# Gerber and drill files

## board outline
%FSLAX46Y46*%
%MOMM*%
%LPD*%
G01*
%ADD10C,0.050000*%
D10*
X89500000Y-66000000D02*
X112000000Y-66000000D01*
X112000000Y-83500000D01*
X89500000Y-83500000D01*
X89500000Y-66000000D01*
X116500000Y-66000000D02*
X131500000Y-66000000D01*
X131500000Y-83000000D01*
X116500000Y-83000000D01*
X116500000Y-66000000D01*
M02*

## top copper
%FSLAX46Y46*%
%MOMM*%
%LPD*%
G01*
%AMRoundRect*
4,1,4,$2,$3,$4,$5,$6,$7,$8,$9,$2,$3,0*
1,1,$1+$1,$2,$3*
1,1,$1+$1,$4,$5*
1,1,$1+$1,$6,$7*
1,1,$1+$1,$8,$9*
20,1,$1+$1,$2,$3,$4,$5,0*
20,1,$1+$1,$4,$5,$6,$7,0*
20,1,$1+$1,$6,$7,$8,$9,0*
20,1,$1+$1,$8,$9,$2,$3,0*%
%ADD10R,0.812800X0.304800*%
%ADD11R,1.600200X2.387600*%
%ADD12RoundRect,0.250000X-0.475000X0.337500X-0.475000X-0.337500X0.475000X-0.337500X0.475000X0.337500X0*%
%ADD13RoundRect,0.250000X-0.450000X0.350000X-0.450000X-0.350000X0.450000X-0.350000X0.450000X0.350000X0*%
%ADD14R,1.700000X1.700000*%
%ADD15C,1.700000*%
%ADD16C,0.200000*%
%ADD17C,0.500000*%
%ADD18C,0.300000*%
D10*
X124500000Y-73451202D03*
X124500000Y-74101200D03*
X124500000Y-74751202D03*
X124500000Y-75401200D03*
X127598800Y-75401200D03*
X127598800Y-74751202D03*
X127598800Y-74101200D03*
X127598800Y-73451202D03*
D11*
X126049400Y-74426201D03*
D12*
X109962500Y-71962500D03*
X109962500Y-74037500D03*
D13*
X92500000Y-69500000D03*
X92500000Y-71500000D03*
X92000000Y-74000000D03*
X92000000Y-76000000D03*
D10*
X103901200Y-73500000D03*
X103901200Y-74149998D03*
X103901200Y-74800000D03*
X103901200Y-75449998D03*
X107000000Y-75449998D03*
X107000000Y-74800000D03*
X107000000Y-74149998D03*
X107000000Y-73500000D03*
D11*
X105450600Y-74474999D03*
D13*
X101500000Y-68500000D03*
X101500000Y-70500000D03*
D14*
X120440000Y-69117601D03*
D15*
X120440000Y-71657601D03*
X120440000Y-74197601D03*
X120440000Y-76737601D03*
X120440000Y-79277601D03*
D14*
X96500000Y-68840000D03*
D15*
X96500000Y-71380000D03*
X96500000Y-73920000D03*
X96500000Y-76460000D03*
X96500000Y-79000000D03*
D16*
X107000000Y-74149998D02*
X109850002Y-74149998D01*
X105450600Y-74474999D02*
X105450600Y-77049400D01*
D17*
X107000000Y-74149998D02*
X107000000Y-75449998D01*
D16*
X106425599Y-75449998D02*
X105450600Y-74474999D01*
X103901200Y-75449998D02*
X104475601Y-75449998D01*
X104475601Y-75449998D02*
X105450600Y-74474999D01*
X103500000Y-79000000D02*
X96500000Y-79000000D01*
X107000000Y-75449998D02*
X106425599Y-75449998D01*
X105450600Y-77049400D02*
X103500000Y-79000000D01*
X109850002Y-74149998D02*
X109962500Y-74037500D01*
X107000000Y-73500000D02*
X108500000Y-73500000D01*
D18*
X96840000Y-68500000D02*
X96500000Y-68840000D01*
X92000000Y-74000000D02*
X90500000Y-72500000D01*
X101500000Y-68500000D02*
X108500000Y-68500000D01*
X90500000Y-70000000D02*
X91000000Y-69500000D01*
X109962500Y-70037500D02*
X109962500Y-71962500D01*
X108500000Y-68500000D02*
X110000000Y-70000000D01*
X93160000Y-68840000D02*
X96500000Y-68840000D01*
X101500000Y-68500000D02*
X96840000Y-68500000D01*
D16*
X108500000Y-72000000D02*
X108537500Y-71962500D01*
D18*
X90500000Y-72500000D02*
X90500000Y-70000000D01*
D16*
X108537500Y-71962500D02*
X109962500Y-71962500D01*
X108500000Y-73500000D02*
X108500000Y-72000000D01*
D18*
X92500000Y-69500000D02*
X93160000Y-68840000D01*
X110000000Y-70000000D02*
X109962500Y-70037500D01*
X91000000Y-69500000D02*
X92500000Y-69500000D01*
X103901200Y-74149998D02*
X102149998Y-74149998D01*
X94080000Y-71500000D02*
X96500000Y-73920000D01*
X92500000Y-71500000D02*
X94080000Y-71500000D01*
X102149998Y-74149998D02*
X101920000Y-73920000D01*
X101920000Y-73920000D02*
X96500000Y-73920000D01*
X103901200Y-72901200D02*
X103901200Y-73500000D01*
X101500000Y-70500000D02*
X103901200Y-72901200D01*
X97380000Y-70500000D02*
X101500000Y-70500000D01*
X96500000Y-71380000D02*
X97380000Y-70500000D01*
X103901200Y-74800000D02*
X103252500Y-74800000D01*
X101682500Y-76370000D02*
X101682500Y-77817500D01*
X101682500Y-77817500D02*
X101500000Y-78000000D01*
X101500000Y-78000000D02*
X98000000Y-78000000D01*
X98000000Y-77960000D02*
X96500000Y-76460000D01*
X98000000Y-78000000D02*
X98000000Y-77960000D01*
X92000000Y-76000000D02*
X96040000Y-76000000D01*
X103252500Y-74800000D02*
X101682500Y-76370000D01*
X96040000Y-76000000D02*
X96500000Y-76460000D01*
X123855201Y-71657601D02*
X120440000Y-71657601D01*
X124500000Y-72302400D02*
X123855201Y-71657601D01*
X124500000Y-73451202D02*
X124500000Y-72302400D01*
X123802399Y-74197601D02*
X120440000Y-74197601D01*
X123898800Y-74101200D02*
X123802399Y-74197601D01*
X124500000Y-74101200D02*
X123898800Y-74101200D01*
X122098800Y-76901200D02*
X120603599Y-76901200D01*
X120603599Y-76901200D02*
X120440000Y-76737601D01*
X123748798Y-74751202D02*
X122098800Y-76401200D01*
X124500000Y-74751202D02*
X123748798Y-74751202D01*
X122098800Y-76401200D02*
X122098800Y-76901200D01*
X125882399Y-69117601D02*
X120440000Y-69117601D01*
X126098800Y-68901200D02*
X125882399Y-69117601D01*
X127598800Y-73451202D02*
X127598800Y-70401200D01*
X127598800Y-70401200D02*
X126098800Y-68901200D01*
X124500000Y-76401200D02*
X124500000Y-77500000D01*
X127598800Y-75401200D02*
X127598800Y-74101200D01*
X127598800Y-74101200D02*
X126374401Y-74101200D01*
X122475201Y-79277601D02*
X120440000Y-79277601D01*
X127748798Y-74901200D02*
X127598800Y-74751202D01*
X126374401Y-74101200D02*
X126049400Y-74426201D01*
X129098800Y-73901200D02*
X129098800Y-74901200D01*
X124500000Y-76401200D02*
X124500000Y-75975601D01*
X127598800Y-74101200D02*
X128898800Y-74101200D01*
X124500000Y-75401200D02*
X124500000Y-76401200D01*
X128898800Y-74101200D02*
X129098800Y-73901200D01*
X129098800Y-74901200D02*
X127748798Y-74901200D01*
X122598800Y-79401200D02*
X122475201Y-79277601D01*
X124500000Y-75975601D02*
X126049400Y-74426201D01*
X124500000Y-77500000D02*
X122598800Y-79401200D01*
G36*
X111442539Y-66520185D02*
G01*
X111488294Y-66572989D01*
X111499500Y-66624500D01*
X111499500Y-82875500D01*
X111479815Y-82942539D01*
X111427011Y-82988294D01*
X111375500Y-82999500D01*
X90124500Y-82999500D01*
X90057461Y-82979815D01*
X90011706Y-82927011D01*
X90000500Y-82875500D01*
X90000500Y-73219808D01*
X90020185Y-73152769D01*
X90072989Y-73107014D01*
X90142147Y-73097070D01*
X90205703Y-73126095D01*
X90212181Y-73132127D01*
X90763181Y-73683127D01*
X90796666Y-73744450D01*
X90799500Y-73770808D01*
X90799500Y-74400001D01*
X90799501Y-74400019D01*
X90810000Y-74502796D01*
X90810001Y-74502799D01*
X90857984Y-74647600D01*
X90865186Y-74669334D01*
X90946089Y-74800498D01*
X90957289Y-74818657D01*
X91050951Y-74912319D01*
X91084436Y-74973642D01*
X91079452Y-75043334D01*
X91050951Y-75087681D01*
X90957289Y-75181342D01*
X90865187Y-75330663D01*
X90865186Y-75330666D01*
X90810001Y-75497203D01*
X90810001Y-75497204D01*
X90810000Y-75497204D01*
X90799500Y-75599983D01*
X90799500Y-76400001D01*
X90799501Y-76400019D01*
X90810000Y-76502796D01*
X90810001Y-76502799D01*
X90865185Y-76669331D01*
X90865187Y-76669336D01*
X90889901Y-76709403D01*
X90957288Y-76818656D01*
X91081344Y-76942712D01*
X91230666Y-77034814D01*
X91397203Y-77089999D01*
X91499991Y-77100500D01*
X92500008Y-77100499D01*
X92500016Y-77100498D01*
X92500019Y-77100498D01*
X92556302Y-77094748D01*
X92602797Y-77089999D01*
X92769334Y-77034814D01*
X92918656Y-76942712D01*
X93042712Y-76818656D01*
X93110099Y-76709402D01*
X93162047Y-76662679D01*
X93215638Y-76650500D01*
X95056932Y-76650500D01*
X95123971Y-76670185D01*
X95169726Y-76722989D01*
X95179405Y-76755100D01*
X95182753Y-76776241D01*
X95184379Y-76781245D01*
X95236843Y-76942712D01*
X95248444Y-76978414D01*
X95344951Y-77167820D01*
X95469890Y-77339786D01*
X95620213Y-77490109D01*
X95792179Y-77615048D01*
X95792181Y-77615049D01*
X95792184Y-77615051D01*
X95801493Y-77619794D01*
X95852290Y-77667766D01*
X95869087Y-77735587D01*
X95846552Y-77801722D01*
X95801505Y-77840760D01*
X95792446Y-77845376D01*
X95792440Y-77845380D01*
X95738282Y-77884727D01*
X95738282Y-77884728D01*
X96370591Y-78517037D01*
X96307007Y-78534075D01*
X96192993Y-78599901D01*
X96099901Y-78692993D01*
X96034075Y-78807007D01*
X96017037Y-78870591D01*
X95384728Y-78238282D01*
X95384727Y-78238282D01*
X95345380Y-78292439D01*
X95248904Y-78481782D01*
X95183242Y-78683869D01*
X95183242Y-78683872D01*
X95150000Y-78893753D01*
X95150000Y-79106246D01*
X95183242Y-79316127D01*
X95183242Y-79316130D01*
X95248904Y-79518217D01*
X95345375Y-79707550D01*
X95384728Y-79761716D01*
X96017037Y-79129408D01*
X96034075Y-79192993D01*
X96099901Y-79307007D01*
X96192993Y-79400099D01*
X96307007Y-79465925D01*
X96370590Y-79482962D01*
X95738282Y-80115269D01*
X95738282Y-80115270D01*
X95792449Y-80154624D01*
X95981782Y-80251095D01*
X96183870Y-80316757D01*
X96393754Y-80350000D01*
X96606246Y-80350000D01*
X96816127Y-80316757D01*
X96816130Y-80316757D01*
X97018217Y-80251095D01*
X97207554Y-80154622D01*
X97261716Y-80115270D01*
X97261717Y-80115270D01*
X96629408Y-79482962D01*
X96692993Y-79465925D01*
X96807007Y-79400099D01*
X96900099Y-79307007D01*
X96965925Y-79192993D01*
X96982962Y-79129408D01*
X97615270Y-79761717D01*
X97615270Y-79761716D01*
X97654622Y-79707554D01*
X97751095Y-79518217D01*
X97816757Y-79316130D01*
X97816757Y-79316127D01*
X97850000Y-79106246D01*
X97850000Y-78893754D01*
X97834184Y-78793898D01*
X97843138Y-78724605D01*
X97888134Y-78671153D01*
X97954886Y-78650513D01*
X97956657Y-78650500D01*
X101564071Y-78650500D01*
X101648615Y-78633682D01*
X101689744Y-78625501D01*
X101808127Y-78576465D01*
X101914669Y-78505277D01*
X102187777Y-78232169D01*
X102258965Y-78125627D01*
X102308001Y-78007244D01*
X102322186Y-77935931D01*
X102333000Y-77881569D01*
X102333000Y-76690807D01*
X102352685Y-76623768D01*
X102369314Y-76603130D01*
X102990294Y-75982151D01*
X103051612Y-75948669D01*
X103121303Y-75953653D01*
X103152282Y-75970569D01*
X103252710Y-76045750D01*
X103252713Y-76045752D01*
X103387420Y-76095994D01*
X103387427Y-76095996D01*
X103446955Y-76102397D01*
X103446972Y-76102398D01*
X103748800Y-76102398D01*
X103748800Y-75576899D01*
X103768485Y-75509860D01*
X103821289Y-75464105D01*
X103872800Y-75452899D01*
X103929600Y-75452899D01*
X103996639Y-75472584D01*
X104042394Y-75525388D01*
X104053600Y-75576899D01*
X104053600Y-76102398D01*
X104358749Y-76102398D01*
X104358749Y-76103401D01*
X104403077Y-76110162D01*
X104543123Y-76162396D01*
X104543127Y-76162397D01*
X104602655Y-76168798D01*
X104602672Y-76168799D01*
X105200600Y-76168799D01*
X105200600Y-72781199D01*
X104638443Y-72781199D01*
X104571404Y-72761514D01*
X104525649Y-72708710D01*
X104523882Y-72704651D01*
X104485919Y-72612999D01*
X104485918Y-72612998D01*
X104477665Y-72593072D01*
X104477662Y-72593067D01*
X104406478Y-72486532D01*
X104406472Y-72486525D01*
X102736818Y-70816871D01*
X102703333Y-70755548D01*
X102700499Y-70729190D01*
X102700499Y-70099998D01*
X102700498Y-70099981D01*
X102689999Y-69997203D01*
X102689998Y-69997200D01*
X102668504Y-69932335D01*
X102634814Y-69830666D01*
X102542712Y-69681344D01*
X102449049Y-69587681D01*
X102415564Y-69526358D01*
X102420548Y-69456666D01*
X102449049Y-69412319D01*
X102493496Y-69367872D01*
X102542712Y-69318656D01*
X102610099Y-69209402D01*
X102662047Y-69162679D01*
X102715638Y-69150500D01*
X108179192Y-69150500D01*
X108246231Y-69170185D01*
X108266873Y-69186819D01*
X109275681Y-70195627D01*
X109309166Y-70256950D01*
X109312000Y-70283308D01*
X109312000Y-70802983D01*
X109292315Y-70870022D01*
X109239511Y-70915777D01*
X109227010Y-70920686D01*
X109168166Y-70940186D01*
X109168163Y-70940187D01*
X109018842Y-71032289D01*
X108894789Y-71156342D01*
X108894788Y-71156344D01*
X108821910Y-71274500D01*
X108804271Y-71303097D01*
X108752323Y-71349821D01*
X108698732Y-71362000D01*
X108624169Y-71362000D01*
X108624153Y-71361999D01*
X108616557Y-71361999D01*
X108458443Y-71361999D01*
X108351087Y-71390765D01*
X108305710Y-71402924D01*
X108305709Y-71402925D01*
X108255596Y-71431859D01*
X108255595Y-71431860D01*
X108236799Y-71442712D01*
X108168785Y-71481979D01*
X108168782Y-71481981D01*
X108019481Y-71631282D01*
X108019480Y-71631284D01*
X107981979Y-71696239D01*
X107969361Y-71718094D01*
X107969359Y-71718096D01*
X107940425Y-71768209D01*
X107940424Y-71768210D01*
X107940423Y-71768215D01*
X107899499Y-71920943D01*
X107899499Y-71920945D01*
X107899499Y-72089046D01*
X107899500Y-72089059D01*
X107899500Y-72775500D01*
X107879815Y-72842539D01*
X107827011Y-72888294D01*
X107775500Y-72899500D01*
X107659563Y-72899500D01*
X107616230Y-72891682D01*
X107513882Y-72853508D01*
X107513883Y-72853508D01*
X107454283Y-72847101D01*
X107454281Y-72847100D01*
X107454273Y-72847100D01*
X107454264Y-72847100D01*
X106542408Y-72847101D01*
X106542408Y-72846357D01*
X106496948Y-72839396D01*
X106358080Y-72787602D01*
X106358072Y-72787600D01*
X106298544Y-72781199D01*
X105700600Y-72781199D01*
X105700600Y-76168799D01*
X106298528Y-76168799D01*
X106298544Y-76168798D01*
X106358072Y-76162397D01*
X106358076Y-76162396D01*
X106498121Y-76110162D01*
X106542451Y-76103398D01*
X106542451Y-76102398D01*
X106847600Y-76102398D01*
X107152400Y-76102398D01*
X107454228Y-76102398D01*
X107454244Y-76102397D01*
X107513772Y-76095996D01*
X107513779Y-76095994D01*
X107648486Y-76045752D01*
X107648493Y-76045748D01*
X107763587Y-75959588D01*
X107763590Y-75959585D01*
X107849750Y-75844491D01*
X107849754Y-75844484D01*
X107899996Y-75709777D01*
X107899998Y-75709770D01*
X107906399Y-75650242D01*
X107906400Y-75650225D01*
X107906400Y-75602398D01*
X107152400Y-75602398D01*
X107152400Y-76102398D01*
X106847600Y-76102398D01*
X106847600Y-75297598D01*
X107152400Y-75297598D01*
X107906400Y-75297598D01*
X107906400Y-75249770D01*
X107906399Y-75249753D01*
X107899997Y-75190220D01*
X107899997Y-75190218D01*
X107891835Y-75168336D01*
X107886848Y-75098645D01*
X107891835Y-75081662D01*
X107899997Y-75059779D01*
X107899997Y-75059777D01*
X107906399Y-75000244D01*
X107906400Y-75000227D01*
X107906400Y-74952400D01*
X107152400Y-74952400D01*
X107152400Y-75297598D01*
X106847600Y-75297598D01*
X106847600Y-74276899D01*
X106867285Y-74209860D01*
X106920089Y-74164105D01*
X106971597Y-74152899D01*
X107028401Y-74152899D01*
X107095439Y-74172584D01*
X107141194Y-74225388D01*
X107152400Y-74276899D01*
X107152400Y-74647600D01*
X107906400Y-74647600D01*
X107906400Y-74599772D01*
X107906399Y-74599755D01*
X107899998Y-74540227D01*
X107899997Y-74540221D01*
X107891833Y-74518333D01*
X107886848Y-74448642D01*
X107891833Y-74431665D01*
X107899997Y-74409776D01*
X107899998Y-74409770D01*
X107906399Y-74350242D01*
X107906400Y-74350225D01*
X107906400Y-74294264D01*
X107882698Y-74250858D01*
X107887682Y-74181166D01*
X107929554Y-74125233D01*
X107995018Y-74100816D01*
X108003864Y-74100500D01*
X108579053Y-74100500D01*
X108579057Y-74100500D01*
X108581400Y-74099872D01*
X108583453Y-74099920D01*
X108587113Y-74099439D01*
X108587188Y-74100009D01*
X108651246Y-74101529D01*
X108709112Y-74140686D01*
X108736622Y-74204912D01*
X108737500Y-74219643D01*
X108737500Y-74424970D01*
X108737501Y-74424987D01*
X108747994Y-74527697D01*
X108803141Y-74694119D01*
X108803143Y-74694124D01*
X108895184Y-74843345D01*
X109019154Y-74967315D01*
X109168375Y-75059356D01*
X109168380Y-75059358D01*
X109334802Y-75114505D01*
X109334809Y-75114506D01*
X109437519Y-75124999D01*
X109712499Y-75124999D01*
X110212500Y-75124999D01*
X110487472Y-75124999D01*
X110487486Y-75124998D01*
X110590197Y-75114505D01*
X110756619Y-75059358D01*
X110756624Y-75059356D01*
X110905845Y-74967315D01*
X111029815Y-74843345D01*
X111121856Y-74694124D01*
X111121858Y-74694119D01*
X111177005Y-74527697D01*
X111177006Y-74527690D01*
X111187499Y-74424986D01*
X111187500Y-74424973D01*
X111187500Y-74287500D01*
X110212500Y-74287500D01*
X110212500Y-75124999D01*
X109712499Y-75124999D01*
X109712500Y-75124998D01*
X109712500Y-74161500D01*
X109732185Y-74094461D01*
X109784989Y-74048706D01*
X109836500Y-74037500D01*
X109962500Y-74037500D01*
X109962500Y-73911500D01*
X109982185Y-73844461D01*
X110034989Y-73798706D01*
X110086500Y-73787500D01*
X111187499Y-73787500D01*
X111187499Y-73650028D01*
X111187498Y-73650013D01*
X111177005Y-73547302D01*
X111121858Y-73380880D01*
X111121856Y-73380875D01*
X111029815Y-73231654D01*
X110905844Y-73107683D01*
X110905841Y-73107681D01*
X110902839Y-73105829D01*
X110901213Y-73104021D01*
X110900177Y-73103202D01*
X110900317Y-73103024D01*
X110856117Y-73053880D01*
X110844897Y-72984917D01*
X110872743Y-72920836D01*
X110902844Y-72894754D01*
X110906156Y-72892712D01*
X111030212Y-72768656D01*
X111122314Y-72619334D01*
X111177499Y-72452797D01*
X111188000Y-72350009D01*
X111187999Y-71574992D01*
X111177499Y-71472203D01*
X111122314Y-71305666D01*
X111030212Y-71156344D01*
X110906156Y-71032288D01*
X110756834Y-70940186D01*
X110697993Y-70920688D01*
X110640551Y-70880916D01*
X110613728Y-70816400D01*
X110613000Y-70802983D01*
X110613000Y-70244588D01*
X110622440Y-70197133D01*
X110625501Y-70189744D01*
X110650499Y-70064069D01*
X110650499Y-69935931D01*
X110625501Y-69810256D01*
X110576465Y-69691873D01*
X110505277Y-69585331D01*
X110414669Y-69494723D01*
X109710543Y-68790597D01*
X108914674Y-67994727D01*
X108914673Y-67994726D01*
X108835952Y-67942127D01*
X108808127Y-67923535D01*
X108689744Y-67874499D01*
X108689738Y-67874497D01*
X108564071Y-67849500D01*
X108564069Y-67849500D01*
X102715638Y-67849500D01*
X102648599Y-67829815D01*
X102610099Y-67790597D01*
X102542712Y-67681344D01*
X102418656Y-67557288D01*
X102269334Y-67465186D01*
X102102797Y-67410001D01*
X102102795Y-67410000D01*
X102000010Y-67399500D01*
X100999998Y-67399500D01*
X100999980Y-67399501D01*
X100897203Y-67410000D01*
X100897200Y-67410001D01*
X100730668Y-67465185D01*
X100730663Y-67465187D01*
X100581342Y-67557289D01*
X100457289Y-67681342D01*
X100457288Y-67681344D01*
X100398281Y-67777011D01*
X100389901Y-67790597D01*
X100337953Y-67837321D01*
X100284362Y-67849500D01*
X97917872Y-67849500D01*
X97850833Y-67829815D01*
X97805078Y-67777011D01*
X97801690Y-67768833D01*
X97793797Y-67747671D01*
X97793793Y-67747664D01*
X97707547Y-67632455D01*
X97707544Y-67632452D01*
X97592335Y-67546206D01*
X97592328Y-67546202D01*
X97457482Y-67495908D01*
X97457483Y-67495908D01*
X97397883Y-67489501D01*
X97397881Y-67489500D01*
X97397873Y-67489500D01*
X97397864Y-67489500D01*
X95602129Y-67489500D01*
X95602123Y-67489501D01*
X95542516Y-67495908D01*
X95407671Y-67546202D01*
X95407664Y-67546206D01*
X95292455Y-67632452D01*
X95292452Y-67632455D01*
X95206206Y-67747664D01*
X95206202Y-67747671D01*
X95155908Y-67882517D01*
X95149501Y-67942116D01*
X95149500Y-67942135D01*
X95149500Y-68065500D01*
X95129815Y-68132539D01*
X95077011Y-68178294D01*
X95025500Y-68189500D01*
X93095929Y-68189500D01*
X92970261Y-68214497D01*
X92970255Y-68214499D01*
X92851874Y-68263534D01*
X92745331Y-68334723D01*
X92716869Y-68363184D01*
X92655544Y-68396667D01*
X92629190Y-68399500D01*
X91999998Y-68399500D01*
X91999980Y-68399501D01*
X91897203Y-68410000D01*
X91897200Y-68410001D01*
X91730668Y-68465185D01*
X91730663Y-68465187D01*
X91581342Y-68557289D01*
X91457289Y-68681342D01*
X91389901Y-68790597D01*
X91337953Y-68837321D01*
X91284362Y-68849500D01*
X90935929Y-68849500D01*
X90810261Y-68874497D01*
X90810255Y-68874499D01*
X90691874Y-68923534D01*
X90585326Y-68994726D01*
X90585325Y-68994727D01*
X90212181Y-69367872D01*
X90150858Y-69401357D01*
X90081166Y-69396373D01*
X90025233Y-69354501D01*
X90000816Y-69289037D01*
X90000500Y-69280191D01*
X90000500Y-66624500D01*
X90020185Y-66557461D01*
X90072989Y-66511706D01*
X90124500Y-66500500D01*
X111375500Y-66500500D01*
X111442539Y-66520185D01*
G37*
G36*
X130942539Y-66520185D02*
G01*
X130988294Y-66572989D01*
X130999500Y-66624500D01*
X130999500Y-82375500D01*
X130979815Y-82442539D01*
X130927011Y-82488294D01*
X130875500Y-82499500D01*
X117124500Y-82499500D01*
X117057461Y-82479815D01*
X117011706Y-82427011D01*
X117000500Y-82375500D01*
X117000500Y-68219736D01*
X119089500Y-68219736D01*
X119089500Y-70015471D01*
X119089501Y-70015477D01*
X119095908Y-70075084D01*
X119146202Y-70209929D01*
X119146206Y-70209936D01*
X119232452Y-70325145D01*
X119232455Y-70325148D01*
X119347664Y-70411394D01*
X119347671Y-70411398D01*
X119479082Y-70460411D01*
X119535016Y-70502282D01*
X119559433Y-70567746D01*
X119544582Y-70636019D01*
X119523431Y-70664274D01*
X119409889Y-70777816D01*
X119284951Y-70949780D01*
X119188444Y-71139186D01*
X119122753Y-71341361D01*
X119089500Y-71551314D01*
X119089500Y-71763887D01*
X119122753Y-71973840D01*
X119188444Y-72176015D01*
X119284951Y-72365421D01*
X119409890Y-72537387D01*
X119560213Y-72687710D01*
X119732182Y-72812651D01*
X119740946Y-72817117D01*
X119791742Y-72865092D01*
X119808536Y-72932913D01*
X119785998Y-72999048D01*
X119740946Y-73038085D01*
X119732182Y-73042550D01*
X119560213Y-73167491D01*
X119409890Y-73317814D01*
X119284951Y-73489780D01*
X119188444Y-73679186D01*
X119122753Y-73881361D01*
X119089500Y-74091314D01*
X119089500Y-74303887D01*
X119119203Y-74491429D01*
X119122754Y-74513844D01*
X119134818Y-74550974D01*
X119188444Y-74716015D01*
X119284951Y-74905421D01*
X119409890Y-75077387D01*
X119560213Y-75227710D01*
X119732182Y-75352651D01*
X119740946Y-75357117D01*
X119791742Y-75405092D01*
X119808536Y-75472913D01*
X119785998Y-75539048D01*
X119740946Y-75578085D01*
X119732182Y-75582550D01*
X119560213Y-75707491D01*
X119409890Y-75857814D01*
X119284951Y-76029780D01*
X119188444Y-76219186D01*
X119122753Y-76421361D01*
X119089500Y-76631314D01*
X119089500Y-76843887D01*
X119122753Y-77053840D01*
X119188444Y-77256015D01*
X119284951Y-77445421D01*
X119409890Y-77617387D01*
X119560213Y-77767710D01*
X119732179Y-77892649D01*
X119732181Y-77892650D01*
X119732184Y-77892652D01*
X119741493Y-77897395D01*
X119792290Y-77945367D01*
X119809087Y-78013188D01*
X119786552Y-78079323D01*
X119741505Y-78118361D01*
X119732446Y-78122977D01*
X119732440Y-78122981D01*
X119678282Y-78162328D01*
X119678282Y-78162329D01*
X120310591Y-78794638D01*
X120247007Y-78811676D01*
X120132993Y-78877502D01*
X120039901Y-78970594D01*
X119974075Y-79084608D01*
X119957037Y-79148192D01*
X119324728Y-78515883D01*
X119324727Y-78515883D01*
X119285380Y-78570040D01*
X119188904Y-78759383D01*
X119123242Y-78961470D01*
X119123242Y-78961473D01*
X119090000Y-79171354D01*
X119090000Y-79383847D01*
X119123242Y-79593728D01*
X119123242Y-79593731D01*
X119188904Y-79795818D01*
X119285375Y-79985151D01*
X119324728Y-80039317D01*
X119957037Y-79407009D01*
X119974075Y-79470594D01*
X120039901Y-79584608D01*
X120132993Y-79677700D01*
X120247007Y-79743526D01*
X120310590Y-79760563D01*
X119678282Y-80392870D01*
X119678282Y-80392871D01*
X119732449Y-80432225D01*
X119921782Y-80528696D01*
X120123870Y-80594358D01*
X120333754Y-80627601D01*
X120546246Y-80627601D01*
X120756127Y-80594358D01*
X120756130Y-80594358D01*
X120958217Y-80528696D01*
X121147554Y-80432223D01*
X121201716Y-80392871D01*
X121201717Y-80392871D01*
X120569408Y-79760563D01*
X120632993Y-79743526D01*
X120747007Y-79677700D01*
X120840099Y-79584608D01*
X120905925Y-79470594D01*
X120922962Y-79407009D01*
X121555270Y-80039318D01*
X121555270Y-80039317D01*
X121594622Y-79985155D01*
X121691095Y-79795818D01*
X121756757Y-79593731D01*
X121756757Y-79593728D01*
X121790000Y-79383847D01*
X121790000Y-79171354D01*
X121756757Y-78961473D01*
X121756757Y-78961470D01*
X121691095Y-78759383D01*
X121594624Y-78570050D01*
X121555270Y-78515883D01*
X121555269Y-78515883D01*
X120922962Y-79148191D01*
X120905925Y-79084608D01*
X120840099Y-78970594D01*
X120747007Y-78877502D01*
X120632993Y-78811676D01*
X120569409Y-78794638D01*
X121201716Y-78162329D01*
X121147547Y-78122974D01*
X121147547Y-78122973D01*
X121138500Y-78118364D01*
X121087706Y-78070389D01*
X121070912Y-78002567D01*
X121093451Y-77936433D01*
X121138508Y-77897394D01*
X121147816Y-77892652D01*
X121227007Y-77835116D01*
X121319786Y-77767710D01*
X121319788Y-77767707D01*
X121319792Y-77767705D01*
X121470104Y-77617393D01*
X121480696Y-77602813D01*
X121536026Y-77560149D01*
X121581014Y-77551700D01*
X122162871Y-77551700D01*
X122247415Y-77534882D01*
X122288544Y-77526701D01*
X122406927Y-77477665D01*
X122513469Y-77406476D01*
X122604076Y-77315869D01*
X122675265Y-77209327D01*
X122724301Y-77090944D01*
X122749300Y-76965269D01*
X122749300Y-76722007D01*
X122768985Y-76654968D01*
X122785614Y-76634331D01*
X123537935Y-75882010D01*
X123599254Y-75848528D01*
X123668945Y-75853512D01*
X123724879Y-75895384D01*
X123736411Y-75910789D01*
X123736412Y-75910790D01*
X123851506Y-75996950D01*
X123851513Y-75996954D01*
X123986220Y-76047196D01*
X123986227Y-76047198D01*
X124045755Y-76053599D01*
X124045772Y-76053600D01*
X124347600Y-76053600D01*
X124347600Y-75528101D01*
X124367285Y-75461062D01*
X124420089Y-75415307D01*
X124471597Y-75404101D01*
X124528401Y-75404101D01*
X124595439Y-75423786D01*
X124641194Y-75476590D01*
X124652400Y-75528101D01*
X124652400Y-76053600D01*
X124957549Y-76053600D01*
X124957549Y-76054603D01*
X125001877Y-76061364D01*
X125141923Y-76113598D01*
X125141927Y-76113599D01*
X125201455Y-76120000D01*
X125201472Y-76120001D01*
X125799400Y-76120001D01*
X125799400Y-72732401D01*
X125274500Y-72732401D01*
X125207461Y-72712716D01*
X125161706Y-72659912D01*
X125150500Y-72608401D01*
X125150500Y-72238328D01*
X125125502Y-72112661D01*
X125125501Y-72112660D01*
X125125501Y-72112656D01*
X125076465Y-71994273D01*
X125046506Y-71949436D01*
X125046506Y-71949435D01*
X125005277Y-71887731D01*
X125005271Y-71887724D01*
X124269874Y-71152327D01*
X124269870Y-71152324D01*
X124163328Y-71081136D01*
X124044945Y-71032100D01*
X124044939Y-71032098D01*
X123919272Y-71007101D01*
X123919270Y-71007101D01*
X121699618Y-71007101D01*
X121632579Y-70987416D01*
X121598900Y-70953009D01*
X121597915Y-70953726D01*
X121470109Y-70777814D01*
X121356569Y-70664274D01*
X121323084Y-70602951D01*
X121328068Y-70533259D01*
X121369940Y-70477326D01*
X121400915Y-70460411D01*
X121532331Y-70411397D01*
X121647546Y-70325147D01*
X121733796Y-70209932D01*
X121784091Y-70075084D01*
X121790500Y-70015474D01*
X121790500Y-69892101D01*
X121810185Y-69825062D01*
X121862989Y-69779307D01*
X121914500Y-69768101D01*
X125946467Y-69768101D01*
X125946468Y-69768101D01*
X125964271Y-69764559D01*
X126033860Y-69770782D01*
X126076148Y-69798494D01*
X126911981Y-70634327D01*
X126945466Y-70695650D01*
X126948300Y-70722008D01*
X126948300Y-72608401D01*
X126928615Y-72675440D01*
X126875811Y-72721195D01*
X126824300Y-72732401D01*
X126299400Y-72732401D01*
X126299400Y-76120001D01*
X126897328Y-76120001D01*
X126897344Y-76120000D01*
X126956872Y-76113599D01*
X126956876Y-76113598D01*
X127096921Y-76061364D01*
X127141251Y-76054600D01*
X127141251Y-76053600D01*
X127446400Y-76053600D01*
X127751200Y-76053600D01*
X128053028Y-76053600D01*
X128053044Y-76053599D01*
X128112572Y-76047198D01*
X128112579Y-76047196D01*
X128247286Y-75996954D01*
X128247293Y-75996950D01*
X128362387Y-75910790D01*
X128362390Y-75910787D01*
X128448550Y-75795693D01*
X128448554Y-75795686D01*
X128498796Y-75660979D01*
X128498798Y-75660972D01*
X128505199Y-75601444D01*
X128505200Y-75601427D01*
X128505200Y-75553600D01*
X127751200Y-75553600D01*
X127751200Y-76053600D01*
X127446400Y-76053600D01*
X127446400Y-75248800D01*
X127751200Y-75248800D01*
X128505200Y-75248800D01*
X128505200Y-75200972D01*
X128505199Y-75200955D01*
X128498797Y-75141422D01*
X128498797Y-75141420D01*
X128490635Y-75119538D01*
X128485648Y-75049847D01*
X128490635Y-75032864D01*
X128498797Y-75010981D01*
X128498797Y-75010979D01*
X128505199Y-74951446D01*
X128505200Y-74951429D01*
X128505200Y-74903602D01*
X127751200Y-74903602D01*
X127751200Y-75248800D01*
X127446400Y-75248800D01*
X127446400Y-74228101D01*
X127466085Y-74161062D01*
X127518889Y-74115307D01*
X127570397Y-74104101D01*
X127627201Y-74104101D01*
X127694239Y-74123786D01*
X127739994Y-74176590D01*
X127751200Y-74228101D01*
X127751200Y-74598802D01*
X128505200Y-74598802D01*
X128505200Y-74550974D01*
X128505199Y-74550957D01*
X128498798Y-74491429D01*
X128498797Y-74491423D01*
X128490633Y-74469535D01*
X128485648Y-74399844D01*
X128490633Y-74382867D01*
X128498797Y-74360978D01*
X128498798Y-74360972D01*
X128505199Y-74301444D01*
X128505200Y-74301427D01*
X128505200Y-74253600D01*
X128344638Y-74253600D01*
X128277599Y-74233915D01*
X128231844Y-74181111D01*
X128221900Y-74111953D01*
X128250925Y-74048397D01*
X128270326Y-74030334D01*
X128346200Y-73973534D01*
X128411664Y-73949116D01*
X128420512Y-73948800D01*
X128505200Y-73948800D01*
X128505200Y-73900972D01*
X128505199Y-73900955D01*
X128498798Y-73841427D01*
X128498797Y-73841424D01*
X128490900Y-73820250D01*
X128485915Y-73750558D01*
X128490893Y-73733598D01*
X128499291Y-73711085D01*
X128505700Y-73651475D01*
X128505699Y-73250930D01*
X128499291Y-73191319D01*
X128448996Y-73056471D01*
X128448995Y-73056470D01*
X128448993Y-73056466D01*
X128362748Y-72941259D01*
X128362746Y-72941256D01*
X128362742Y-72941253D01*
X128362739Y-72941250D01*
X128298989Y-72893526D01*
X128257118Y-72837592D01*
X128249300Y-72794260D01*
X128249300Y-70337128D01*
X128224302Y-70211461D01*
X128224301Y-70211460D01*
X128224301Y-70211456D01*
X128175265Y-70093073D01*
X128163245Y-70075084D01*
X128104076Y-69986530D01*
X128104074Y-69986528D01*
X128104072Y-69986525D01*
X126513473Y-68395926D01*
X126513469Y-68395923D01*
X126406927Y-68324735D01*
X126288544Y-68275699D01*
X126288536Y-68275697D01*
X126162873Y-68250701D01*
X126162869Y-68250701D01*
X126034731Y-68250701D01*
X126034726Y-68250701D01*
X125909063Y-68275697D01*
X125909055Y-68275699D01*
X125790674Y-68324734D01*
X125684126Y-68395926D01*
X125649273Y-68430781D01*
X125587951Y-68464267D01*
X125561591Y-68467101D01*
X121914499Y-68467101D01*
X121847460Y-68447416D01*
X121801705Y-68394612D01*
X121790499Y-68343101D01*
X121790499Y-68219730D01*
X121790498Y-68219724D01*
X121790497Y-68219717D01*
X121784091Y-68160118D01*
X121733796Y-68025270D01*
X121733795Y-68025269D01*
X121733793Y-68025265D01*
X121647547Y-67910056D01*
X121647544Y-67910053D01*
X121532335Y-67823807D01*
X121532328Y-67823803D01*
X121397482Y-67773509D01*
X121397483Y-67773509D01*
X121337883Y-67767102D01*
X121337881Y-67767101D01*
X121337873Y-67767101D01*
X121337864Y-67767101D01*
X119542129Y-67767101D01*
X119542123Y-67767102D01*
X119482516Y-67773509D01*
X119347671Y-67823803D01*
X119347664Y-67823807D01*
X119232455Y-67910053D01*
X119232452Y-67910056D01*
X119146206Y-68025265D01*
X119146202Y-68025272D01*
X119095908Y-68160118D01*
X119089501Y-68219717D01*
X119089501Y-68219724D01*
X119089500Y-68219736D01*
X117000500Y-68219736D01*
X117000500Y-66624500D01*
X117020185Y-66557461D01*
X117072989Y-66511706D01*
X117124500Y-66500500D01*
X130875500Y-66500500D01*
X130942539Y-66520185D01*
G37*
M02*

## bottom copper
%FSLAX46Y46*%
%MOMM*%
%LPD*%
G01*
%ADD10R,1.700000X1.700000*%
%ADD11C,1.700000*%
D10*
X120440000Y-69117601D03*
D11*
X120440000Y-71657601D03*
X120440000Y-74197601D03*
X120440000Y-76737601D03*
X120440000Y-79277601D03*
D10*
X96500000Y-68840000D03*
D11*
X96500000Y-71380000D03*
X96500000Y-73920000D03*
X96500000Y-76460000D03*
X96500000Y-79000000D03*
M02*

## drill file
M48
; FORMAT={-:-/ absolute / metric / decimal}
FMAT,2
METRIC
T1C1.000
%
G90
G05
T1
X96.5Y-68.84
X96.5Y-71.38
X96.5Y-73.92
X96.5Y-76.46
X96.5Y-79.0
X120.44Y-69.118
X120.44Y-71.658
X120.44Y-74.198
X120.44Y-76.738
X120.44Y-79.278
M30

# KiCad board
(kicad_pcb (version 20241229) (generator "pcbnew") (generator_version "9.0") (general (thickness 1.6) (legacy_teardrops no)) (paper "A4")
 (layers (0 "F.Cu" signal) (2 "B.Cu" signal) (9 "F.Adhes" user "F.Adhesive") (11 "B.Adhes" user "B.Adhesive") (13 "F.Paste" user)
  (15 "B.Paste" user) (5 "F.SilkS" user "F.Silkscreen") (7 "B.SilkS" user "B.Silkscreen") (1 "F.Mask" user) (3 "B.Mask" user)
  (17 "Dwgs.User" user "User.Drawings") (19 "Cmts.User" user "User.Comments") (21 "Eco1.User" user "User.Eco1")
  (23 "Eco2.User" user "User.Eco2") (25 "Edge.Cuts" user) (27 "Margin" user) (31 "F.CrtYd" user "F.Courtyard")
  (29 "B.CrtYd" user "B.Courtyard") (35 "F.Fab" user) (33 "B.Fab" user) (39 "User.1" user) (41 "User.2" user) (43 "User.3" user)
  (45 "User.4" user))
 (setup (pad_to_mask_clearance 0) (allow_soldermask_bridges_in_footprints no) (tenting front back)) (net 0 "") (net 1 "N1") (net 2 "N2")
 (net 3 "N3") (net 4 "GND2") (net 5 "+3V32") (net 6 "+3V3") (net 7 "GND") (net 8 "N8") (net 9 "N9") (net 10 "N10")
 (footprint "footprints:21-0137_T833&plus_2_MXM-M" (layer "F.Cu") (at 126.0494 74.426201)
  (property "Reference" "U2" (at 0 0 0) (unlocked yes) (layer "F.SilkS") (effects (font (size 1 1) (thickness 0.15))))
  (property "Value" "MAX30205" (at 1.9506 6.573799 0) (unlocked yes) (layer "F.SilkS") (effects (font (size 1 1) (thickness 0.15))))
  (pad "1" smd rect (at -1.5494 -0.974999) (size 0.8128 0.3048) (layers "F.Cu" "F.Mask" "F.Paste") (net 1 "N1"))
  (pad "2" smd rect (at -1.5494 -0.325001) (size 0.8128 0.3048) (layers "F.Cu" "F.Mask" "F.Paste") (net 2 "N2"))
  (pad "3" smd rect (at -1.5494 0.325001) (size 0.8128 0.3048) (layers "F.Cu" "F.Mask" "F.Paste") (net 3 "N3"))
  (pad "4" smd rect (at -1.5494 0.974999) (size 0.8128 0.3048) (layers "F.Cu" "F.Mask" "F.Paste") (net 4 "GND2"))
  (pad "5" smd rect (at 1.5494 0.974999) (size 0.8128 0.3048) (layers "F.Cu" "F.Mask" "F.Paste") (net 4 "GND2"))
  (pad "6" smd rect (at 1.5494 0.325001) (size 0.8128 0.3048) (layers "F.Cu" "F.Mask" "F.Paste") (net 4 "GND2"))
  (pad "7" smd rect (at 1.5494 -0.325001) (size 0.8128 0.3048) (layers "F.Cu" "F.Mask" "F.Paste") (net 4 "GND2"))
  (pad "8" smd rect (at 1.5494 -0.974999) (size 0.8128 0.3048) (layers "F.Cu" "F.Mask" "F.Paste") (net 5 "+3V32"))
  (pad "9" smd rect (at 0 0) (size 1.6002 2.3876) (layers "F.Cu" "F.Mask" "F.Paste") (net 4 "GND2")))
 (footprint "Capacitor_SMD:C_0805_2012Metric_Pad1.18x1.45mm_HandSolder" (layer "F.Cu") (at 109.9625 73 -90)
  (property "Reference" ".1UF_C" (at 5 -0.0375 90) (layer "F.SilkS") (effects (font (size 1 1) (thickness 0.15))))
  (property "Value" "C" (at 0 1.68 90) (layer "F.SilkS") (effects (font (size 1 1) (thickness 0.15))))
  (pad "1" smd roundrect (at -1.0375 0 270) (size 1.175 1.45) (layers "F.Cu" "F.Mask" "F.Paste") (roundrect_rratio 0.212766) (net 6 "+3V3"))
  (pad "2" smd roundrect (at 1.0375 0 270) (size 1.175 1.45) (layers "F.Cu" "F.Mask" "F.Paste") (roundrect_rratio 0.212766) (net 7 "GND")))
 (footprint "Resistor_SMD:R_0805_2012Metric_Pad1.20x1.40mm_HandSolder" (layer "F.Cu") (at 92.5 70.5 -90)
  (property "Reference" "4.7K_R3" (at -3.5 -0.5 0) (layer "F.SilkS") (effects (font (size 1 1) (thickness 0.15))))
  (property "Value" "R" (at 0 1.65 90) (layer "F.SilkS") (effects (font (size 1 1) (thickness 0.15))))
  (pad "1" smd roundrect (at -1 0 270) (size 1.2 1.4) (layers "F.Cu" "F.Mask" "F.Paste") (roundrect_rratio 0.208333) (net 6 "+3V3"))
  (pad "2" smd roundrect (at 1 0 270) (size 1.2 1.4) (layers "F.Cu" "F.Mask" "F.Paste") (roundrect_rratio 0.208333) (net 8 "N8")))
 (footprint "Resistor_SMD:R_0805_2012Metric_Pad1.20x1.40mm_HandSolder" (layer "F.Cu") (at 92 75 -90)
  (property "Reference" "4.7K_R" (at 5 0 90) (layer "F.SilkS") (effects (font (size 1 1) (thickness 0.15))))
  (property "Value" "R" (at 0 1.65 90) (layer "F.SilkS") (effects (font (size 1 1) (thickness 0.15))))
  (pad "1" smd roundrect (at -1 0 270) (size 1.2 1.4) (layers "F.Cu" "F.Mask" "F.Paste") (roundrect_rratio 0.208333) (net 6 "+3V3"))
  (pad "2" smd roundrect (at 1 0 270) (size 1.2 1.4) (layers "F.Cu" "F.Mask" "F.Paste") (roundrect_rratio 0.208333) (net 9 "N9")))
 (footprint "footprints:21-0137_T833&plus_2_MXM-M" (layer "F.Cu") (at 105.4506 74.474999)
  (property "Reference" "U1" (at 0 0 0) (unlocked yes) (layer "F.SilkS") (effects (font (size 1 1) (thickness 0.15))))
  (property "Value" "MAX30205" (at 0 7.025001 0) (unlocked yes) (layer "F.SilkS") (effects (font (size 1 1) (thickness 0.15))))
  (pad "1" smd rect (at -1.5494 -0.974999) (size 0.8128 0.3048) (layers "F.Cu" "F.Mask" "F.Paste") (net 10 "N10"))
  (pad "2" smd rect (at -1.5494 -0.325001) (size 0.8128 0.3048) (layers "F.Cu" "F.Mask" "F.Paste") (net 8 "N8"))
  (pad "3" smd rect (at -1.5494 0.325001) (size 0.8128 0.3048) (layers "F.Cu" "F.Mask" "F.Paste") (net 9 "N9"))
  (pad "4" smd rect (at -1.5494 0.974999) (size 0.8128 0.3048) (layers "F.Cu" "F.Mask" "F.Paste") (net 7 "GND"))
  (pad "5" smd rect (at 1.5494 0.974999) (size 0.8128 0.3048) (layers "F.Cu" "F.Mask" "F.Paste") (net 7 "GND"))
  (pad "6" smd rect (at 1.5494 0.325001) (size 0.8128 0.3048) (layers "F.Cu" "F.Mask" "F.Paste") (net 7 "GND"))
  (pad "7" smd rect (at 1.5494 -0.325001) (size 0.8128 0.3048) (layers "F.Cu" "F.Mask" "F.Paste") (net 7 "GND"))
  (pad "8" smd rect (at 1.5494 -0.974999) (size 0.8128 0.3048) (layers "F.Cu" "F.Mask" "F.Paste") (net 6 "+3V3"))
  (pad "9" smd rect (at 0 0) (size 1.6002 2.3876) (layers "F.Cu" "F.Mask" "F.Paste") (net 7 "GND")))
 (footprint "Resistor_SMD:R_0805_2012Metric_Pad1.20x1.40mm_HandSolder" (layer "F.Cu") (at 101.5 69.5 -90)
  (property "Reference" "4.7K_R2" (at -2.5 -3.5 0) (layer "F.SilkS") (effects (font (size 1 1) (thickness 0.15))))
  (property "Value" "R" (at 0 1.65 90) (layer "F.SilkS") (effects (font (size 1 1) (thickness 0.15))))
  (pad "1" smd roundrect (at -1 0 270) (size 1.2 1.4) (layers "F.Cu" "F.Mask" "F.Paste") (roundrect_rratio 0.208333) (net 6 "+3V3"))
  (pad "2" smd roundrect (at 1 0 270) (size 1.2 1.4) (layers "F.Cu" "F.Mask" "F.Paste") (roundrect_rratio 0.208333) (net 10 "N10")))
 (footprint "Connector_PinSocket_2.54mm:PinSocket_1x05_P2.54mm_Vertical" (layer "F.Cu") (at 120.44 69.117601)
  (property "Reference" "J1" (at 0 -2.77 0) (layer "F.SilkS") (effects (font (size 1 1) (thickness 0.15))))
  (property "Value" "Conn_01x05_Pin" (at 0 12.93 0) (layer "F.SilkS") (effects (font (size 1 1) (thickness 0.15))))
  (pad "1" thru_hole rect (at 0 0) (size 1.7 1.7) (drill 1) (layers "*.Cu" "*.Mask") (remove_unused_layers no) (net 5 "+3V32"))
  (pad "2" thru_hole circle (at 0 2.54) (size 1.7 1.7) (drill 1) (layers "*.Cu" "*.Mask") (remove_unused_layers no) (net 1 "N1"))
  (pad "3" thru_hole circle (at 0 5.08) (size 1.7 1.7) (drill 1) (layers "*.Cu" "*.Mask") (remove_unused_layers no) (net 2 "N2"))
  (pad "4" thru_hole circle (at 0 7.62) (size 1.7 1.7) (drill 1) (layers "*.Cu" "*.Mask") (remove_unused_layers no) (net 3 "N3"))
  (pad "5" thru_hole circle (at 0 10.16) (size 1.7 1.7) (drill 1) (layers "*.Cu" "*.Mask") (remove_unused_layers no) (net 4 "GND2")))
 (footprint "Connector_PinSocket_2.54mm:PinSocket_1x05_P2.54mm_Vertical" (layer "F.Cu") (at 96.5 68.84)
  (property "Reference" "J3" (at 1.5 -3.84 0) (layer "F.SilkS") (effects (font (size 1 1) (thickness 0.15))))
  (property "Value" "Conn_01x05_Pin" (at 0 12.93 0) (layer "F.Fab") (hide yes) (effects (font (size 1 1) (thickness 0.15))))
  (pad "1" thru_hole rect (at 0 0) (size 1.7 1.7) (drill 1) (layers "*.Cu" "*.Mask") (remove_unused_layers no) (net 6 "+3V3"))
  (pad "2" thru_hole circle (at 0 2.54) (size 1.7 1.7) (drill 1) (layers "*.Cu" "*.Mask") (remove_unused_layers no) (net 10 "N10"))
  (pad "3" thru_hole circle (at 0 5.08) (size 1.7 1.7) (drill 1) (layers "*.Cu" "*.Mask") (remove_unused_layers no) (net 8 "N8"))
  (pad "4" thru_hole circle (at 0 7.62) (size 1.7 1.7) (drill 1) (layers "*.Cu" "*.Mask") (remove_unused_layers no) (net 9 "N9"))
  (pad "5" thru_hole circle (at 0 10.16) (size 1.7 1.7) (drill 1) (layers "*.Cu" "*.Mask") (remove_unused_layers no) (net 7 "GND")))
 (gr_rect (start 89.5 66) (end 112 83.5) (stroke (width 0.05) (type default)) (fill no) (layer "Edge.Cuts"))
 (gr_rect (start 116.5 66) (end 131.5 83) (stroke (width 0.05) (type default)) (fill no) (layer "Edge.Cuts"))
 (segment (start 107 74.149998) (end 109.850002 74.149998) (width 0.2) (layer "F.Cu") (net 7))
 (segment (start 105.4506 74.474999) (end 105.4506 77.0494) (width 0.2) (layer "F.Cu") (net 7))
 (segment (start 107 74.149998) (end 107 75.449998) (width 0.5) (layer "F.Cu") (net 7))
 (segment (start 106.425599 75.449998) (end 105.4506 74.474999) (width 0.2) (layer "F.Cu") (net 7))
 (segment (start 103.9012 75.449998) (end 104.475601 75.449998) (width 0.2) (layer "F.Cu") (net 7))
 (segment (start 104.475601 75.449998) (end 105.4506 74.474999) (width 0.2) (layer "F.Cu") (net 7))
 (segment (start 103.5 79) (end 96.5 79) (width 0.2) (layer "F.Cu") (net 7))
 (segment (start 107 75.449998) (end 106.425599 75.449998) (width 0.2) (layer "F.Cu") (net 7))
 (segment (start 105.4506 77.0494) (end 103.5 79) (width 0.2) (layer "F.Cu") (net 7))
 (segment (start 109.850002 74.149998) (end 109.9625 74.0375) (width 0.2) (layer "F.Cu") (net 7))
 (segment (start 107 73.5) (end 108.5 73.5) (width 0.2) (layer "F.Cu") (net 6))
 (segment (start 96.84 68.5) (end 96.5 68.84) (width 0.3) (layer "F.Cu") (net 6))
 (segment (start 92 74) (end 90.5 72.5) (width 0.3) (layer "F.Cu") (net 6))
 (segment (start 101.5 68.5) (end 108.5 68.5) (width 0.3) (layer "F.Cu") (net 6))
 (segment (start 90.5 70) (end 91 69.5) (width 0.3) (layer "F.Cu") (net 6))
 (segment (start 109.9625 70.0375) (end 109.9625 71.9625) (width 0.3) (layer "F.Cu") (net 6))
 (segment (start 108.5 68.5) (end 110 70) (width 0.3) (layer "F.Cu") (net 6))
 (segment (start 93.16 68.84) (end 96.5 68.84) (width 0.3) (layer "F.Cu") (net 6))
 (segment (start 101.5 68.5) (end 96.84 68.5) (width 0.3) (layer "F.Cu") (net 6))
 (segment (start 108.5 72) (end 108.5375 71.9625) (width 0.2) (layer "F.Cu") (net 6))
 (segment (start 90.5 72.5) (end 90.5 70) (width 0.3) (layer "F.Cu") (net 6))
 (segment (start 108.5375 71.9625) (end 109.9625 71.9625) (width 0.2) (layer "F.Cu") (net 6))
 (segment (start 108.5 73.5) (end 108.5 72) (width 0.2) (layer "F.Cu") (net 6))
 (segment (start 92.5 69.5) (end 93.16 68.84) (width 0.3) (layer "F.Cu") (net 6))
 (segment (start 110 70) (end 109.9625 70.0375) (width 0.3) (layer "F.Cu") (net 6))
 (segment (start 91 69.5) (end 92.5 69.5) (width 0.3) (layer "F.Cu") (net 6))
 (segment (start 103.9012 74.149998) (end 102.149998 74.149998) (width 0.3) (layer "F.Cu") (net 8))
 (segment (start 94.08 71.5) (end 96.5 73.92) (width 0.3) (layer "F.Cu") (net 8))
 (segment (start 92.5 71.5) (end 94.08 71.5) (width 0.3) (layer "F.Cu") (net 8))
 (segment (start 102.149998 74.149998) (end 101.92 73.92) (width 0.3) (layer "F.Cu") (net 8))
 (segment (start 101.92 73.92) (end 96.5 73.92) (width 0.3) (layer "F.Cu") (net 8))
 (segment (start 103.9012 72.9012) (end 103.9012 73.5) (width 0.3) (layer "F.Cu") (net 10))
 (segment (start 101.5 70.5) (end 103.9012 72.9012) (width 0.3) (layer "F.Cu") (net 10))
 (segment (start 97.38 70.5) (end 101.5 70.5) (width 0.3) (layer "F.Cu") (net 10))
 (segment (start 96.5 71.38) (end 97.38 70.5) (width 0.3) (layer "F.Cu") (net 10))
 (segment (start 103.9012 74.8) (end 103.2525 74.8) (width 0.3) (layer "F.Cu") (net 9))
 (segment (start 101.6825 76.37) (end 101.6825 77.8175) (width 0.3) (layer "F.Cu") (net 9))
 (segment (start 101.6825 77.8175) (end 101.5 78) (width 0.3) (layer "F.Cu") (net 9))
 (segment (start 101.5 78) (end 98 78) (width 0.3) (layer "F.Cu") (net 9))
 (segment (start 98 77.96) (end 96.5 76.46) (width 0.3) (layer "F.Cu") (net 9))
 (segment (start 98 78) (end 98 77.96) (width 0.3) (layer "F.Cu") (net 9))
 (segment (start 92 76) (end 96.04 76) (width 0.3) (layer "F.Cu") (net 9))
 (segment (start 103.2525 74.8) (end 101.6825 76.37) (width 0.3) (layer "F.Cu") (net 9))
 (segment (start 96.04 76) (end 96.5 76.46) (width 0.3) (layer "F.Cu") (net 9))
 (segment (start 123.855201 71.657601) (end 120.44 71.657601) (width 0.3) (layer "F.Cu") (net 1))
 (segment (start 124.5 72.3024) (end 123.855201 71.657601) (width 0.3) (layer "F.Cu") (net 1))
 (segment (start 124.5 73.451202) (end 124.5 72.3024) (width 0.3) (layer "F.Cu") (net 1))
 (segment (start 123.802399 74.197601) (end 120.44 74.197601) (width 0.3) (layer "F.Cu") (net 2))
 (segment (start 123.8988 74.1012) (end 123.802399 74.197601) (width 0.3) (layer "F.Cu") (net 2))
 (segment (start 124.5 74.1012) (end 123.8988 74.1012) (width 0.3) (layer "F.Cu") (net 2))
 (segment (start 122.0988 76.9012) (end 120.603599 76.9012) (width 0.3) (layer "F.Cu") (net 3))
 (segment (start 120.603599 76.9012) (end 120.44 76.737601) (width 0.3) (layer "F.Cu") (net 3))
 (segment (start 123.748798 74.751202) (end 122.0988 76.4012) (width 0.3) (layer "F.Cu") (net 3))
 (segment (start 124.5 74.751202) (end 123.748798 74.751202) (width 0.3) (layer "F.Cu") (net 3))
 (segment (start 122.0988 76.4012) (end 122.0988 76.9012) (width 0.3) (layer "F.Cu") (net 3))
 (segment (start 125.882399 69.117601) (end 120.44 69.117601) (width 0.3) (layer "F.Cu") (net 5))
 (segment (start 126.0988 68.9012) (end 125.882399 69.117601) (width 0.3) (layer "F.Cu") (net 5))
 (segment (start 127.5988 73.451202) (end 127.5988 70.4012) (width 0.3) (layer "F.Cu") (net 5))
 (segment (start 127.5988 70.4012) (end 126.0988 68.9012) (width 0.3) (layer "F.Cu") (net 5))
 (segment (start 124.5 76.4012) (end 124.5 77.5) (width 0.3) (layer "F.Cu") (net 4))
 (segment (start 127.5988 75.4012) (end 127.5988 74.1012) (width 0.3) (layer "F.Cu") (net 4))
 (segment (start 127.5988 74.1012) (end 126.374401 74.1012) (width 0.3) (layer "F.Cu") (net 4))
 (segment (start 122.475201 79.277601) (end 120.44 79.277601) (width 0.3) (layer "F.Cu") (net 4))
 (segment (start 127.748798 74.9012) (end 127.5988 74.751202) (width 0.3) (layer "F.Cu") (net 4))
 (segment (start 126.374401 74.1012) (end 126.0494 74.426201) (width 0.3) (layer "F.Cu") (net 4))
 (segment (start 129.0988 73.9012) (end 129.0988 74.9012) (width 0.3) (layer "F.Cu") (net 4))
 (segment (start 124.5 76.4012) (end 124.5 75.975601) (width 0.3) (layer "F.Cu") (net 4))
 (segment (start 127.5988 74.1012) (end 128.8988 74.1012) (width 0.3) (layer "F.Cu") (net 4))
 (segment (start 124.5 75.4012) (end 124.5 76.4012) (width 0.3) (layer "F.Cu") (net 4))
 (segment (start 128.8988 74.1012) (end 129.0988 73.9012) (width 0.3) (layer "F.Cu") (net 4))
 (segment (start 129.0988 74.9012) (end 127.748798 74.9012) (width 0.3) (layer "F.Cu") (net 4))
 (segment (start 122.5988 79.4012) (end 122.475201 79.277601) (width 0.3) (layer "F.Cu") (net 4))
 (segment (start 124.5 75.975601) (end 126.0494 74.426201) (width 0.3) (layer "F.Cu") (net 4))
 (segment (start 124.5 77.5) (end 122.5988 79.4012) (width 0.3) (layer "F.Cu") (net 4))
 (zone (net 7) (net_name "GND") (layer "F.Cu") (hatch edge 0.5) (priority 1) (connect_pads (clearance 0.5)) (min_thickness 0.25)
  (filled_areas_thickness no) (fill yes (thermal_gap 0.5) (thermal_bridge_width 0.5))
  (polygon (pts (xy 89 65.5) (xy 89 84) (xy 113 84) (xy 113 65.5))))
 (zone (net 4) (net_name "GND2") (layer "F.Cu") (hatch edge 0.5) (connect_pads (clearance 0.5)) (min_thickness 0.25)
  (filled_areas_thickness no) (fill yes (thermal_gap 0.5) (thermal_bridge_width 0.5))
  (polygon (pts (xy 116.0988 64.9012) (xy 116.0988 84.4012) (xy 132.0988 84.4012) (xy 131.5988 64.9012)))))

